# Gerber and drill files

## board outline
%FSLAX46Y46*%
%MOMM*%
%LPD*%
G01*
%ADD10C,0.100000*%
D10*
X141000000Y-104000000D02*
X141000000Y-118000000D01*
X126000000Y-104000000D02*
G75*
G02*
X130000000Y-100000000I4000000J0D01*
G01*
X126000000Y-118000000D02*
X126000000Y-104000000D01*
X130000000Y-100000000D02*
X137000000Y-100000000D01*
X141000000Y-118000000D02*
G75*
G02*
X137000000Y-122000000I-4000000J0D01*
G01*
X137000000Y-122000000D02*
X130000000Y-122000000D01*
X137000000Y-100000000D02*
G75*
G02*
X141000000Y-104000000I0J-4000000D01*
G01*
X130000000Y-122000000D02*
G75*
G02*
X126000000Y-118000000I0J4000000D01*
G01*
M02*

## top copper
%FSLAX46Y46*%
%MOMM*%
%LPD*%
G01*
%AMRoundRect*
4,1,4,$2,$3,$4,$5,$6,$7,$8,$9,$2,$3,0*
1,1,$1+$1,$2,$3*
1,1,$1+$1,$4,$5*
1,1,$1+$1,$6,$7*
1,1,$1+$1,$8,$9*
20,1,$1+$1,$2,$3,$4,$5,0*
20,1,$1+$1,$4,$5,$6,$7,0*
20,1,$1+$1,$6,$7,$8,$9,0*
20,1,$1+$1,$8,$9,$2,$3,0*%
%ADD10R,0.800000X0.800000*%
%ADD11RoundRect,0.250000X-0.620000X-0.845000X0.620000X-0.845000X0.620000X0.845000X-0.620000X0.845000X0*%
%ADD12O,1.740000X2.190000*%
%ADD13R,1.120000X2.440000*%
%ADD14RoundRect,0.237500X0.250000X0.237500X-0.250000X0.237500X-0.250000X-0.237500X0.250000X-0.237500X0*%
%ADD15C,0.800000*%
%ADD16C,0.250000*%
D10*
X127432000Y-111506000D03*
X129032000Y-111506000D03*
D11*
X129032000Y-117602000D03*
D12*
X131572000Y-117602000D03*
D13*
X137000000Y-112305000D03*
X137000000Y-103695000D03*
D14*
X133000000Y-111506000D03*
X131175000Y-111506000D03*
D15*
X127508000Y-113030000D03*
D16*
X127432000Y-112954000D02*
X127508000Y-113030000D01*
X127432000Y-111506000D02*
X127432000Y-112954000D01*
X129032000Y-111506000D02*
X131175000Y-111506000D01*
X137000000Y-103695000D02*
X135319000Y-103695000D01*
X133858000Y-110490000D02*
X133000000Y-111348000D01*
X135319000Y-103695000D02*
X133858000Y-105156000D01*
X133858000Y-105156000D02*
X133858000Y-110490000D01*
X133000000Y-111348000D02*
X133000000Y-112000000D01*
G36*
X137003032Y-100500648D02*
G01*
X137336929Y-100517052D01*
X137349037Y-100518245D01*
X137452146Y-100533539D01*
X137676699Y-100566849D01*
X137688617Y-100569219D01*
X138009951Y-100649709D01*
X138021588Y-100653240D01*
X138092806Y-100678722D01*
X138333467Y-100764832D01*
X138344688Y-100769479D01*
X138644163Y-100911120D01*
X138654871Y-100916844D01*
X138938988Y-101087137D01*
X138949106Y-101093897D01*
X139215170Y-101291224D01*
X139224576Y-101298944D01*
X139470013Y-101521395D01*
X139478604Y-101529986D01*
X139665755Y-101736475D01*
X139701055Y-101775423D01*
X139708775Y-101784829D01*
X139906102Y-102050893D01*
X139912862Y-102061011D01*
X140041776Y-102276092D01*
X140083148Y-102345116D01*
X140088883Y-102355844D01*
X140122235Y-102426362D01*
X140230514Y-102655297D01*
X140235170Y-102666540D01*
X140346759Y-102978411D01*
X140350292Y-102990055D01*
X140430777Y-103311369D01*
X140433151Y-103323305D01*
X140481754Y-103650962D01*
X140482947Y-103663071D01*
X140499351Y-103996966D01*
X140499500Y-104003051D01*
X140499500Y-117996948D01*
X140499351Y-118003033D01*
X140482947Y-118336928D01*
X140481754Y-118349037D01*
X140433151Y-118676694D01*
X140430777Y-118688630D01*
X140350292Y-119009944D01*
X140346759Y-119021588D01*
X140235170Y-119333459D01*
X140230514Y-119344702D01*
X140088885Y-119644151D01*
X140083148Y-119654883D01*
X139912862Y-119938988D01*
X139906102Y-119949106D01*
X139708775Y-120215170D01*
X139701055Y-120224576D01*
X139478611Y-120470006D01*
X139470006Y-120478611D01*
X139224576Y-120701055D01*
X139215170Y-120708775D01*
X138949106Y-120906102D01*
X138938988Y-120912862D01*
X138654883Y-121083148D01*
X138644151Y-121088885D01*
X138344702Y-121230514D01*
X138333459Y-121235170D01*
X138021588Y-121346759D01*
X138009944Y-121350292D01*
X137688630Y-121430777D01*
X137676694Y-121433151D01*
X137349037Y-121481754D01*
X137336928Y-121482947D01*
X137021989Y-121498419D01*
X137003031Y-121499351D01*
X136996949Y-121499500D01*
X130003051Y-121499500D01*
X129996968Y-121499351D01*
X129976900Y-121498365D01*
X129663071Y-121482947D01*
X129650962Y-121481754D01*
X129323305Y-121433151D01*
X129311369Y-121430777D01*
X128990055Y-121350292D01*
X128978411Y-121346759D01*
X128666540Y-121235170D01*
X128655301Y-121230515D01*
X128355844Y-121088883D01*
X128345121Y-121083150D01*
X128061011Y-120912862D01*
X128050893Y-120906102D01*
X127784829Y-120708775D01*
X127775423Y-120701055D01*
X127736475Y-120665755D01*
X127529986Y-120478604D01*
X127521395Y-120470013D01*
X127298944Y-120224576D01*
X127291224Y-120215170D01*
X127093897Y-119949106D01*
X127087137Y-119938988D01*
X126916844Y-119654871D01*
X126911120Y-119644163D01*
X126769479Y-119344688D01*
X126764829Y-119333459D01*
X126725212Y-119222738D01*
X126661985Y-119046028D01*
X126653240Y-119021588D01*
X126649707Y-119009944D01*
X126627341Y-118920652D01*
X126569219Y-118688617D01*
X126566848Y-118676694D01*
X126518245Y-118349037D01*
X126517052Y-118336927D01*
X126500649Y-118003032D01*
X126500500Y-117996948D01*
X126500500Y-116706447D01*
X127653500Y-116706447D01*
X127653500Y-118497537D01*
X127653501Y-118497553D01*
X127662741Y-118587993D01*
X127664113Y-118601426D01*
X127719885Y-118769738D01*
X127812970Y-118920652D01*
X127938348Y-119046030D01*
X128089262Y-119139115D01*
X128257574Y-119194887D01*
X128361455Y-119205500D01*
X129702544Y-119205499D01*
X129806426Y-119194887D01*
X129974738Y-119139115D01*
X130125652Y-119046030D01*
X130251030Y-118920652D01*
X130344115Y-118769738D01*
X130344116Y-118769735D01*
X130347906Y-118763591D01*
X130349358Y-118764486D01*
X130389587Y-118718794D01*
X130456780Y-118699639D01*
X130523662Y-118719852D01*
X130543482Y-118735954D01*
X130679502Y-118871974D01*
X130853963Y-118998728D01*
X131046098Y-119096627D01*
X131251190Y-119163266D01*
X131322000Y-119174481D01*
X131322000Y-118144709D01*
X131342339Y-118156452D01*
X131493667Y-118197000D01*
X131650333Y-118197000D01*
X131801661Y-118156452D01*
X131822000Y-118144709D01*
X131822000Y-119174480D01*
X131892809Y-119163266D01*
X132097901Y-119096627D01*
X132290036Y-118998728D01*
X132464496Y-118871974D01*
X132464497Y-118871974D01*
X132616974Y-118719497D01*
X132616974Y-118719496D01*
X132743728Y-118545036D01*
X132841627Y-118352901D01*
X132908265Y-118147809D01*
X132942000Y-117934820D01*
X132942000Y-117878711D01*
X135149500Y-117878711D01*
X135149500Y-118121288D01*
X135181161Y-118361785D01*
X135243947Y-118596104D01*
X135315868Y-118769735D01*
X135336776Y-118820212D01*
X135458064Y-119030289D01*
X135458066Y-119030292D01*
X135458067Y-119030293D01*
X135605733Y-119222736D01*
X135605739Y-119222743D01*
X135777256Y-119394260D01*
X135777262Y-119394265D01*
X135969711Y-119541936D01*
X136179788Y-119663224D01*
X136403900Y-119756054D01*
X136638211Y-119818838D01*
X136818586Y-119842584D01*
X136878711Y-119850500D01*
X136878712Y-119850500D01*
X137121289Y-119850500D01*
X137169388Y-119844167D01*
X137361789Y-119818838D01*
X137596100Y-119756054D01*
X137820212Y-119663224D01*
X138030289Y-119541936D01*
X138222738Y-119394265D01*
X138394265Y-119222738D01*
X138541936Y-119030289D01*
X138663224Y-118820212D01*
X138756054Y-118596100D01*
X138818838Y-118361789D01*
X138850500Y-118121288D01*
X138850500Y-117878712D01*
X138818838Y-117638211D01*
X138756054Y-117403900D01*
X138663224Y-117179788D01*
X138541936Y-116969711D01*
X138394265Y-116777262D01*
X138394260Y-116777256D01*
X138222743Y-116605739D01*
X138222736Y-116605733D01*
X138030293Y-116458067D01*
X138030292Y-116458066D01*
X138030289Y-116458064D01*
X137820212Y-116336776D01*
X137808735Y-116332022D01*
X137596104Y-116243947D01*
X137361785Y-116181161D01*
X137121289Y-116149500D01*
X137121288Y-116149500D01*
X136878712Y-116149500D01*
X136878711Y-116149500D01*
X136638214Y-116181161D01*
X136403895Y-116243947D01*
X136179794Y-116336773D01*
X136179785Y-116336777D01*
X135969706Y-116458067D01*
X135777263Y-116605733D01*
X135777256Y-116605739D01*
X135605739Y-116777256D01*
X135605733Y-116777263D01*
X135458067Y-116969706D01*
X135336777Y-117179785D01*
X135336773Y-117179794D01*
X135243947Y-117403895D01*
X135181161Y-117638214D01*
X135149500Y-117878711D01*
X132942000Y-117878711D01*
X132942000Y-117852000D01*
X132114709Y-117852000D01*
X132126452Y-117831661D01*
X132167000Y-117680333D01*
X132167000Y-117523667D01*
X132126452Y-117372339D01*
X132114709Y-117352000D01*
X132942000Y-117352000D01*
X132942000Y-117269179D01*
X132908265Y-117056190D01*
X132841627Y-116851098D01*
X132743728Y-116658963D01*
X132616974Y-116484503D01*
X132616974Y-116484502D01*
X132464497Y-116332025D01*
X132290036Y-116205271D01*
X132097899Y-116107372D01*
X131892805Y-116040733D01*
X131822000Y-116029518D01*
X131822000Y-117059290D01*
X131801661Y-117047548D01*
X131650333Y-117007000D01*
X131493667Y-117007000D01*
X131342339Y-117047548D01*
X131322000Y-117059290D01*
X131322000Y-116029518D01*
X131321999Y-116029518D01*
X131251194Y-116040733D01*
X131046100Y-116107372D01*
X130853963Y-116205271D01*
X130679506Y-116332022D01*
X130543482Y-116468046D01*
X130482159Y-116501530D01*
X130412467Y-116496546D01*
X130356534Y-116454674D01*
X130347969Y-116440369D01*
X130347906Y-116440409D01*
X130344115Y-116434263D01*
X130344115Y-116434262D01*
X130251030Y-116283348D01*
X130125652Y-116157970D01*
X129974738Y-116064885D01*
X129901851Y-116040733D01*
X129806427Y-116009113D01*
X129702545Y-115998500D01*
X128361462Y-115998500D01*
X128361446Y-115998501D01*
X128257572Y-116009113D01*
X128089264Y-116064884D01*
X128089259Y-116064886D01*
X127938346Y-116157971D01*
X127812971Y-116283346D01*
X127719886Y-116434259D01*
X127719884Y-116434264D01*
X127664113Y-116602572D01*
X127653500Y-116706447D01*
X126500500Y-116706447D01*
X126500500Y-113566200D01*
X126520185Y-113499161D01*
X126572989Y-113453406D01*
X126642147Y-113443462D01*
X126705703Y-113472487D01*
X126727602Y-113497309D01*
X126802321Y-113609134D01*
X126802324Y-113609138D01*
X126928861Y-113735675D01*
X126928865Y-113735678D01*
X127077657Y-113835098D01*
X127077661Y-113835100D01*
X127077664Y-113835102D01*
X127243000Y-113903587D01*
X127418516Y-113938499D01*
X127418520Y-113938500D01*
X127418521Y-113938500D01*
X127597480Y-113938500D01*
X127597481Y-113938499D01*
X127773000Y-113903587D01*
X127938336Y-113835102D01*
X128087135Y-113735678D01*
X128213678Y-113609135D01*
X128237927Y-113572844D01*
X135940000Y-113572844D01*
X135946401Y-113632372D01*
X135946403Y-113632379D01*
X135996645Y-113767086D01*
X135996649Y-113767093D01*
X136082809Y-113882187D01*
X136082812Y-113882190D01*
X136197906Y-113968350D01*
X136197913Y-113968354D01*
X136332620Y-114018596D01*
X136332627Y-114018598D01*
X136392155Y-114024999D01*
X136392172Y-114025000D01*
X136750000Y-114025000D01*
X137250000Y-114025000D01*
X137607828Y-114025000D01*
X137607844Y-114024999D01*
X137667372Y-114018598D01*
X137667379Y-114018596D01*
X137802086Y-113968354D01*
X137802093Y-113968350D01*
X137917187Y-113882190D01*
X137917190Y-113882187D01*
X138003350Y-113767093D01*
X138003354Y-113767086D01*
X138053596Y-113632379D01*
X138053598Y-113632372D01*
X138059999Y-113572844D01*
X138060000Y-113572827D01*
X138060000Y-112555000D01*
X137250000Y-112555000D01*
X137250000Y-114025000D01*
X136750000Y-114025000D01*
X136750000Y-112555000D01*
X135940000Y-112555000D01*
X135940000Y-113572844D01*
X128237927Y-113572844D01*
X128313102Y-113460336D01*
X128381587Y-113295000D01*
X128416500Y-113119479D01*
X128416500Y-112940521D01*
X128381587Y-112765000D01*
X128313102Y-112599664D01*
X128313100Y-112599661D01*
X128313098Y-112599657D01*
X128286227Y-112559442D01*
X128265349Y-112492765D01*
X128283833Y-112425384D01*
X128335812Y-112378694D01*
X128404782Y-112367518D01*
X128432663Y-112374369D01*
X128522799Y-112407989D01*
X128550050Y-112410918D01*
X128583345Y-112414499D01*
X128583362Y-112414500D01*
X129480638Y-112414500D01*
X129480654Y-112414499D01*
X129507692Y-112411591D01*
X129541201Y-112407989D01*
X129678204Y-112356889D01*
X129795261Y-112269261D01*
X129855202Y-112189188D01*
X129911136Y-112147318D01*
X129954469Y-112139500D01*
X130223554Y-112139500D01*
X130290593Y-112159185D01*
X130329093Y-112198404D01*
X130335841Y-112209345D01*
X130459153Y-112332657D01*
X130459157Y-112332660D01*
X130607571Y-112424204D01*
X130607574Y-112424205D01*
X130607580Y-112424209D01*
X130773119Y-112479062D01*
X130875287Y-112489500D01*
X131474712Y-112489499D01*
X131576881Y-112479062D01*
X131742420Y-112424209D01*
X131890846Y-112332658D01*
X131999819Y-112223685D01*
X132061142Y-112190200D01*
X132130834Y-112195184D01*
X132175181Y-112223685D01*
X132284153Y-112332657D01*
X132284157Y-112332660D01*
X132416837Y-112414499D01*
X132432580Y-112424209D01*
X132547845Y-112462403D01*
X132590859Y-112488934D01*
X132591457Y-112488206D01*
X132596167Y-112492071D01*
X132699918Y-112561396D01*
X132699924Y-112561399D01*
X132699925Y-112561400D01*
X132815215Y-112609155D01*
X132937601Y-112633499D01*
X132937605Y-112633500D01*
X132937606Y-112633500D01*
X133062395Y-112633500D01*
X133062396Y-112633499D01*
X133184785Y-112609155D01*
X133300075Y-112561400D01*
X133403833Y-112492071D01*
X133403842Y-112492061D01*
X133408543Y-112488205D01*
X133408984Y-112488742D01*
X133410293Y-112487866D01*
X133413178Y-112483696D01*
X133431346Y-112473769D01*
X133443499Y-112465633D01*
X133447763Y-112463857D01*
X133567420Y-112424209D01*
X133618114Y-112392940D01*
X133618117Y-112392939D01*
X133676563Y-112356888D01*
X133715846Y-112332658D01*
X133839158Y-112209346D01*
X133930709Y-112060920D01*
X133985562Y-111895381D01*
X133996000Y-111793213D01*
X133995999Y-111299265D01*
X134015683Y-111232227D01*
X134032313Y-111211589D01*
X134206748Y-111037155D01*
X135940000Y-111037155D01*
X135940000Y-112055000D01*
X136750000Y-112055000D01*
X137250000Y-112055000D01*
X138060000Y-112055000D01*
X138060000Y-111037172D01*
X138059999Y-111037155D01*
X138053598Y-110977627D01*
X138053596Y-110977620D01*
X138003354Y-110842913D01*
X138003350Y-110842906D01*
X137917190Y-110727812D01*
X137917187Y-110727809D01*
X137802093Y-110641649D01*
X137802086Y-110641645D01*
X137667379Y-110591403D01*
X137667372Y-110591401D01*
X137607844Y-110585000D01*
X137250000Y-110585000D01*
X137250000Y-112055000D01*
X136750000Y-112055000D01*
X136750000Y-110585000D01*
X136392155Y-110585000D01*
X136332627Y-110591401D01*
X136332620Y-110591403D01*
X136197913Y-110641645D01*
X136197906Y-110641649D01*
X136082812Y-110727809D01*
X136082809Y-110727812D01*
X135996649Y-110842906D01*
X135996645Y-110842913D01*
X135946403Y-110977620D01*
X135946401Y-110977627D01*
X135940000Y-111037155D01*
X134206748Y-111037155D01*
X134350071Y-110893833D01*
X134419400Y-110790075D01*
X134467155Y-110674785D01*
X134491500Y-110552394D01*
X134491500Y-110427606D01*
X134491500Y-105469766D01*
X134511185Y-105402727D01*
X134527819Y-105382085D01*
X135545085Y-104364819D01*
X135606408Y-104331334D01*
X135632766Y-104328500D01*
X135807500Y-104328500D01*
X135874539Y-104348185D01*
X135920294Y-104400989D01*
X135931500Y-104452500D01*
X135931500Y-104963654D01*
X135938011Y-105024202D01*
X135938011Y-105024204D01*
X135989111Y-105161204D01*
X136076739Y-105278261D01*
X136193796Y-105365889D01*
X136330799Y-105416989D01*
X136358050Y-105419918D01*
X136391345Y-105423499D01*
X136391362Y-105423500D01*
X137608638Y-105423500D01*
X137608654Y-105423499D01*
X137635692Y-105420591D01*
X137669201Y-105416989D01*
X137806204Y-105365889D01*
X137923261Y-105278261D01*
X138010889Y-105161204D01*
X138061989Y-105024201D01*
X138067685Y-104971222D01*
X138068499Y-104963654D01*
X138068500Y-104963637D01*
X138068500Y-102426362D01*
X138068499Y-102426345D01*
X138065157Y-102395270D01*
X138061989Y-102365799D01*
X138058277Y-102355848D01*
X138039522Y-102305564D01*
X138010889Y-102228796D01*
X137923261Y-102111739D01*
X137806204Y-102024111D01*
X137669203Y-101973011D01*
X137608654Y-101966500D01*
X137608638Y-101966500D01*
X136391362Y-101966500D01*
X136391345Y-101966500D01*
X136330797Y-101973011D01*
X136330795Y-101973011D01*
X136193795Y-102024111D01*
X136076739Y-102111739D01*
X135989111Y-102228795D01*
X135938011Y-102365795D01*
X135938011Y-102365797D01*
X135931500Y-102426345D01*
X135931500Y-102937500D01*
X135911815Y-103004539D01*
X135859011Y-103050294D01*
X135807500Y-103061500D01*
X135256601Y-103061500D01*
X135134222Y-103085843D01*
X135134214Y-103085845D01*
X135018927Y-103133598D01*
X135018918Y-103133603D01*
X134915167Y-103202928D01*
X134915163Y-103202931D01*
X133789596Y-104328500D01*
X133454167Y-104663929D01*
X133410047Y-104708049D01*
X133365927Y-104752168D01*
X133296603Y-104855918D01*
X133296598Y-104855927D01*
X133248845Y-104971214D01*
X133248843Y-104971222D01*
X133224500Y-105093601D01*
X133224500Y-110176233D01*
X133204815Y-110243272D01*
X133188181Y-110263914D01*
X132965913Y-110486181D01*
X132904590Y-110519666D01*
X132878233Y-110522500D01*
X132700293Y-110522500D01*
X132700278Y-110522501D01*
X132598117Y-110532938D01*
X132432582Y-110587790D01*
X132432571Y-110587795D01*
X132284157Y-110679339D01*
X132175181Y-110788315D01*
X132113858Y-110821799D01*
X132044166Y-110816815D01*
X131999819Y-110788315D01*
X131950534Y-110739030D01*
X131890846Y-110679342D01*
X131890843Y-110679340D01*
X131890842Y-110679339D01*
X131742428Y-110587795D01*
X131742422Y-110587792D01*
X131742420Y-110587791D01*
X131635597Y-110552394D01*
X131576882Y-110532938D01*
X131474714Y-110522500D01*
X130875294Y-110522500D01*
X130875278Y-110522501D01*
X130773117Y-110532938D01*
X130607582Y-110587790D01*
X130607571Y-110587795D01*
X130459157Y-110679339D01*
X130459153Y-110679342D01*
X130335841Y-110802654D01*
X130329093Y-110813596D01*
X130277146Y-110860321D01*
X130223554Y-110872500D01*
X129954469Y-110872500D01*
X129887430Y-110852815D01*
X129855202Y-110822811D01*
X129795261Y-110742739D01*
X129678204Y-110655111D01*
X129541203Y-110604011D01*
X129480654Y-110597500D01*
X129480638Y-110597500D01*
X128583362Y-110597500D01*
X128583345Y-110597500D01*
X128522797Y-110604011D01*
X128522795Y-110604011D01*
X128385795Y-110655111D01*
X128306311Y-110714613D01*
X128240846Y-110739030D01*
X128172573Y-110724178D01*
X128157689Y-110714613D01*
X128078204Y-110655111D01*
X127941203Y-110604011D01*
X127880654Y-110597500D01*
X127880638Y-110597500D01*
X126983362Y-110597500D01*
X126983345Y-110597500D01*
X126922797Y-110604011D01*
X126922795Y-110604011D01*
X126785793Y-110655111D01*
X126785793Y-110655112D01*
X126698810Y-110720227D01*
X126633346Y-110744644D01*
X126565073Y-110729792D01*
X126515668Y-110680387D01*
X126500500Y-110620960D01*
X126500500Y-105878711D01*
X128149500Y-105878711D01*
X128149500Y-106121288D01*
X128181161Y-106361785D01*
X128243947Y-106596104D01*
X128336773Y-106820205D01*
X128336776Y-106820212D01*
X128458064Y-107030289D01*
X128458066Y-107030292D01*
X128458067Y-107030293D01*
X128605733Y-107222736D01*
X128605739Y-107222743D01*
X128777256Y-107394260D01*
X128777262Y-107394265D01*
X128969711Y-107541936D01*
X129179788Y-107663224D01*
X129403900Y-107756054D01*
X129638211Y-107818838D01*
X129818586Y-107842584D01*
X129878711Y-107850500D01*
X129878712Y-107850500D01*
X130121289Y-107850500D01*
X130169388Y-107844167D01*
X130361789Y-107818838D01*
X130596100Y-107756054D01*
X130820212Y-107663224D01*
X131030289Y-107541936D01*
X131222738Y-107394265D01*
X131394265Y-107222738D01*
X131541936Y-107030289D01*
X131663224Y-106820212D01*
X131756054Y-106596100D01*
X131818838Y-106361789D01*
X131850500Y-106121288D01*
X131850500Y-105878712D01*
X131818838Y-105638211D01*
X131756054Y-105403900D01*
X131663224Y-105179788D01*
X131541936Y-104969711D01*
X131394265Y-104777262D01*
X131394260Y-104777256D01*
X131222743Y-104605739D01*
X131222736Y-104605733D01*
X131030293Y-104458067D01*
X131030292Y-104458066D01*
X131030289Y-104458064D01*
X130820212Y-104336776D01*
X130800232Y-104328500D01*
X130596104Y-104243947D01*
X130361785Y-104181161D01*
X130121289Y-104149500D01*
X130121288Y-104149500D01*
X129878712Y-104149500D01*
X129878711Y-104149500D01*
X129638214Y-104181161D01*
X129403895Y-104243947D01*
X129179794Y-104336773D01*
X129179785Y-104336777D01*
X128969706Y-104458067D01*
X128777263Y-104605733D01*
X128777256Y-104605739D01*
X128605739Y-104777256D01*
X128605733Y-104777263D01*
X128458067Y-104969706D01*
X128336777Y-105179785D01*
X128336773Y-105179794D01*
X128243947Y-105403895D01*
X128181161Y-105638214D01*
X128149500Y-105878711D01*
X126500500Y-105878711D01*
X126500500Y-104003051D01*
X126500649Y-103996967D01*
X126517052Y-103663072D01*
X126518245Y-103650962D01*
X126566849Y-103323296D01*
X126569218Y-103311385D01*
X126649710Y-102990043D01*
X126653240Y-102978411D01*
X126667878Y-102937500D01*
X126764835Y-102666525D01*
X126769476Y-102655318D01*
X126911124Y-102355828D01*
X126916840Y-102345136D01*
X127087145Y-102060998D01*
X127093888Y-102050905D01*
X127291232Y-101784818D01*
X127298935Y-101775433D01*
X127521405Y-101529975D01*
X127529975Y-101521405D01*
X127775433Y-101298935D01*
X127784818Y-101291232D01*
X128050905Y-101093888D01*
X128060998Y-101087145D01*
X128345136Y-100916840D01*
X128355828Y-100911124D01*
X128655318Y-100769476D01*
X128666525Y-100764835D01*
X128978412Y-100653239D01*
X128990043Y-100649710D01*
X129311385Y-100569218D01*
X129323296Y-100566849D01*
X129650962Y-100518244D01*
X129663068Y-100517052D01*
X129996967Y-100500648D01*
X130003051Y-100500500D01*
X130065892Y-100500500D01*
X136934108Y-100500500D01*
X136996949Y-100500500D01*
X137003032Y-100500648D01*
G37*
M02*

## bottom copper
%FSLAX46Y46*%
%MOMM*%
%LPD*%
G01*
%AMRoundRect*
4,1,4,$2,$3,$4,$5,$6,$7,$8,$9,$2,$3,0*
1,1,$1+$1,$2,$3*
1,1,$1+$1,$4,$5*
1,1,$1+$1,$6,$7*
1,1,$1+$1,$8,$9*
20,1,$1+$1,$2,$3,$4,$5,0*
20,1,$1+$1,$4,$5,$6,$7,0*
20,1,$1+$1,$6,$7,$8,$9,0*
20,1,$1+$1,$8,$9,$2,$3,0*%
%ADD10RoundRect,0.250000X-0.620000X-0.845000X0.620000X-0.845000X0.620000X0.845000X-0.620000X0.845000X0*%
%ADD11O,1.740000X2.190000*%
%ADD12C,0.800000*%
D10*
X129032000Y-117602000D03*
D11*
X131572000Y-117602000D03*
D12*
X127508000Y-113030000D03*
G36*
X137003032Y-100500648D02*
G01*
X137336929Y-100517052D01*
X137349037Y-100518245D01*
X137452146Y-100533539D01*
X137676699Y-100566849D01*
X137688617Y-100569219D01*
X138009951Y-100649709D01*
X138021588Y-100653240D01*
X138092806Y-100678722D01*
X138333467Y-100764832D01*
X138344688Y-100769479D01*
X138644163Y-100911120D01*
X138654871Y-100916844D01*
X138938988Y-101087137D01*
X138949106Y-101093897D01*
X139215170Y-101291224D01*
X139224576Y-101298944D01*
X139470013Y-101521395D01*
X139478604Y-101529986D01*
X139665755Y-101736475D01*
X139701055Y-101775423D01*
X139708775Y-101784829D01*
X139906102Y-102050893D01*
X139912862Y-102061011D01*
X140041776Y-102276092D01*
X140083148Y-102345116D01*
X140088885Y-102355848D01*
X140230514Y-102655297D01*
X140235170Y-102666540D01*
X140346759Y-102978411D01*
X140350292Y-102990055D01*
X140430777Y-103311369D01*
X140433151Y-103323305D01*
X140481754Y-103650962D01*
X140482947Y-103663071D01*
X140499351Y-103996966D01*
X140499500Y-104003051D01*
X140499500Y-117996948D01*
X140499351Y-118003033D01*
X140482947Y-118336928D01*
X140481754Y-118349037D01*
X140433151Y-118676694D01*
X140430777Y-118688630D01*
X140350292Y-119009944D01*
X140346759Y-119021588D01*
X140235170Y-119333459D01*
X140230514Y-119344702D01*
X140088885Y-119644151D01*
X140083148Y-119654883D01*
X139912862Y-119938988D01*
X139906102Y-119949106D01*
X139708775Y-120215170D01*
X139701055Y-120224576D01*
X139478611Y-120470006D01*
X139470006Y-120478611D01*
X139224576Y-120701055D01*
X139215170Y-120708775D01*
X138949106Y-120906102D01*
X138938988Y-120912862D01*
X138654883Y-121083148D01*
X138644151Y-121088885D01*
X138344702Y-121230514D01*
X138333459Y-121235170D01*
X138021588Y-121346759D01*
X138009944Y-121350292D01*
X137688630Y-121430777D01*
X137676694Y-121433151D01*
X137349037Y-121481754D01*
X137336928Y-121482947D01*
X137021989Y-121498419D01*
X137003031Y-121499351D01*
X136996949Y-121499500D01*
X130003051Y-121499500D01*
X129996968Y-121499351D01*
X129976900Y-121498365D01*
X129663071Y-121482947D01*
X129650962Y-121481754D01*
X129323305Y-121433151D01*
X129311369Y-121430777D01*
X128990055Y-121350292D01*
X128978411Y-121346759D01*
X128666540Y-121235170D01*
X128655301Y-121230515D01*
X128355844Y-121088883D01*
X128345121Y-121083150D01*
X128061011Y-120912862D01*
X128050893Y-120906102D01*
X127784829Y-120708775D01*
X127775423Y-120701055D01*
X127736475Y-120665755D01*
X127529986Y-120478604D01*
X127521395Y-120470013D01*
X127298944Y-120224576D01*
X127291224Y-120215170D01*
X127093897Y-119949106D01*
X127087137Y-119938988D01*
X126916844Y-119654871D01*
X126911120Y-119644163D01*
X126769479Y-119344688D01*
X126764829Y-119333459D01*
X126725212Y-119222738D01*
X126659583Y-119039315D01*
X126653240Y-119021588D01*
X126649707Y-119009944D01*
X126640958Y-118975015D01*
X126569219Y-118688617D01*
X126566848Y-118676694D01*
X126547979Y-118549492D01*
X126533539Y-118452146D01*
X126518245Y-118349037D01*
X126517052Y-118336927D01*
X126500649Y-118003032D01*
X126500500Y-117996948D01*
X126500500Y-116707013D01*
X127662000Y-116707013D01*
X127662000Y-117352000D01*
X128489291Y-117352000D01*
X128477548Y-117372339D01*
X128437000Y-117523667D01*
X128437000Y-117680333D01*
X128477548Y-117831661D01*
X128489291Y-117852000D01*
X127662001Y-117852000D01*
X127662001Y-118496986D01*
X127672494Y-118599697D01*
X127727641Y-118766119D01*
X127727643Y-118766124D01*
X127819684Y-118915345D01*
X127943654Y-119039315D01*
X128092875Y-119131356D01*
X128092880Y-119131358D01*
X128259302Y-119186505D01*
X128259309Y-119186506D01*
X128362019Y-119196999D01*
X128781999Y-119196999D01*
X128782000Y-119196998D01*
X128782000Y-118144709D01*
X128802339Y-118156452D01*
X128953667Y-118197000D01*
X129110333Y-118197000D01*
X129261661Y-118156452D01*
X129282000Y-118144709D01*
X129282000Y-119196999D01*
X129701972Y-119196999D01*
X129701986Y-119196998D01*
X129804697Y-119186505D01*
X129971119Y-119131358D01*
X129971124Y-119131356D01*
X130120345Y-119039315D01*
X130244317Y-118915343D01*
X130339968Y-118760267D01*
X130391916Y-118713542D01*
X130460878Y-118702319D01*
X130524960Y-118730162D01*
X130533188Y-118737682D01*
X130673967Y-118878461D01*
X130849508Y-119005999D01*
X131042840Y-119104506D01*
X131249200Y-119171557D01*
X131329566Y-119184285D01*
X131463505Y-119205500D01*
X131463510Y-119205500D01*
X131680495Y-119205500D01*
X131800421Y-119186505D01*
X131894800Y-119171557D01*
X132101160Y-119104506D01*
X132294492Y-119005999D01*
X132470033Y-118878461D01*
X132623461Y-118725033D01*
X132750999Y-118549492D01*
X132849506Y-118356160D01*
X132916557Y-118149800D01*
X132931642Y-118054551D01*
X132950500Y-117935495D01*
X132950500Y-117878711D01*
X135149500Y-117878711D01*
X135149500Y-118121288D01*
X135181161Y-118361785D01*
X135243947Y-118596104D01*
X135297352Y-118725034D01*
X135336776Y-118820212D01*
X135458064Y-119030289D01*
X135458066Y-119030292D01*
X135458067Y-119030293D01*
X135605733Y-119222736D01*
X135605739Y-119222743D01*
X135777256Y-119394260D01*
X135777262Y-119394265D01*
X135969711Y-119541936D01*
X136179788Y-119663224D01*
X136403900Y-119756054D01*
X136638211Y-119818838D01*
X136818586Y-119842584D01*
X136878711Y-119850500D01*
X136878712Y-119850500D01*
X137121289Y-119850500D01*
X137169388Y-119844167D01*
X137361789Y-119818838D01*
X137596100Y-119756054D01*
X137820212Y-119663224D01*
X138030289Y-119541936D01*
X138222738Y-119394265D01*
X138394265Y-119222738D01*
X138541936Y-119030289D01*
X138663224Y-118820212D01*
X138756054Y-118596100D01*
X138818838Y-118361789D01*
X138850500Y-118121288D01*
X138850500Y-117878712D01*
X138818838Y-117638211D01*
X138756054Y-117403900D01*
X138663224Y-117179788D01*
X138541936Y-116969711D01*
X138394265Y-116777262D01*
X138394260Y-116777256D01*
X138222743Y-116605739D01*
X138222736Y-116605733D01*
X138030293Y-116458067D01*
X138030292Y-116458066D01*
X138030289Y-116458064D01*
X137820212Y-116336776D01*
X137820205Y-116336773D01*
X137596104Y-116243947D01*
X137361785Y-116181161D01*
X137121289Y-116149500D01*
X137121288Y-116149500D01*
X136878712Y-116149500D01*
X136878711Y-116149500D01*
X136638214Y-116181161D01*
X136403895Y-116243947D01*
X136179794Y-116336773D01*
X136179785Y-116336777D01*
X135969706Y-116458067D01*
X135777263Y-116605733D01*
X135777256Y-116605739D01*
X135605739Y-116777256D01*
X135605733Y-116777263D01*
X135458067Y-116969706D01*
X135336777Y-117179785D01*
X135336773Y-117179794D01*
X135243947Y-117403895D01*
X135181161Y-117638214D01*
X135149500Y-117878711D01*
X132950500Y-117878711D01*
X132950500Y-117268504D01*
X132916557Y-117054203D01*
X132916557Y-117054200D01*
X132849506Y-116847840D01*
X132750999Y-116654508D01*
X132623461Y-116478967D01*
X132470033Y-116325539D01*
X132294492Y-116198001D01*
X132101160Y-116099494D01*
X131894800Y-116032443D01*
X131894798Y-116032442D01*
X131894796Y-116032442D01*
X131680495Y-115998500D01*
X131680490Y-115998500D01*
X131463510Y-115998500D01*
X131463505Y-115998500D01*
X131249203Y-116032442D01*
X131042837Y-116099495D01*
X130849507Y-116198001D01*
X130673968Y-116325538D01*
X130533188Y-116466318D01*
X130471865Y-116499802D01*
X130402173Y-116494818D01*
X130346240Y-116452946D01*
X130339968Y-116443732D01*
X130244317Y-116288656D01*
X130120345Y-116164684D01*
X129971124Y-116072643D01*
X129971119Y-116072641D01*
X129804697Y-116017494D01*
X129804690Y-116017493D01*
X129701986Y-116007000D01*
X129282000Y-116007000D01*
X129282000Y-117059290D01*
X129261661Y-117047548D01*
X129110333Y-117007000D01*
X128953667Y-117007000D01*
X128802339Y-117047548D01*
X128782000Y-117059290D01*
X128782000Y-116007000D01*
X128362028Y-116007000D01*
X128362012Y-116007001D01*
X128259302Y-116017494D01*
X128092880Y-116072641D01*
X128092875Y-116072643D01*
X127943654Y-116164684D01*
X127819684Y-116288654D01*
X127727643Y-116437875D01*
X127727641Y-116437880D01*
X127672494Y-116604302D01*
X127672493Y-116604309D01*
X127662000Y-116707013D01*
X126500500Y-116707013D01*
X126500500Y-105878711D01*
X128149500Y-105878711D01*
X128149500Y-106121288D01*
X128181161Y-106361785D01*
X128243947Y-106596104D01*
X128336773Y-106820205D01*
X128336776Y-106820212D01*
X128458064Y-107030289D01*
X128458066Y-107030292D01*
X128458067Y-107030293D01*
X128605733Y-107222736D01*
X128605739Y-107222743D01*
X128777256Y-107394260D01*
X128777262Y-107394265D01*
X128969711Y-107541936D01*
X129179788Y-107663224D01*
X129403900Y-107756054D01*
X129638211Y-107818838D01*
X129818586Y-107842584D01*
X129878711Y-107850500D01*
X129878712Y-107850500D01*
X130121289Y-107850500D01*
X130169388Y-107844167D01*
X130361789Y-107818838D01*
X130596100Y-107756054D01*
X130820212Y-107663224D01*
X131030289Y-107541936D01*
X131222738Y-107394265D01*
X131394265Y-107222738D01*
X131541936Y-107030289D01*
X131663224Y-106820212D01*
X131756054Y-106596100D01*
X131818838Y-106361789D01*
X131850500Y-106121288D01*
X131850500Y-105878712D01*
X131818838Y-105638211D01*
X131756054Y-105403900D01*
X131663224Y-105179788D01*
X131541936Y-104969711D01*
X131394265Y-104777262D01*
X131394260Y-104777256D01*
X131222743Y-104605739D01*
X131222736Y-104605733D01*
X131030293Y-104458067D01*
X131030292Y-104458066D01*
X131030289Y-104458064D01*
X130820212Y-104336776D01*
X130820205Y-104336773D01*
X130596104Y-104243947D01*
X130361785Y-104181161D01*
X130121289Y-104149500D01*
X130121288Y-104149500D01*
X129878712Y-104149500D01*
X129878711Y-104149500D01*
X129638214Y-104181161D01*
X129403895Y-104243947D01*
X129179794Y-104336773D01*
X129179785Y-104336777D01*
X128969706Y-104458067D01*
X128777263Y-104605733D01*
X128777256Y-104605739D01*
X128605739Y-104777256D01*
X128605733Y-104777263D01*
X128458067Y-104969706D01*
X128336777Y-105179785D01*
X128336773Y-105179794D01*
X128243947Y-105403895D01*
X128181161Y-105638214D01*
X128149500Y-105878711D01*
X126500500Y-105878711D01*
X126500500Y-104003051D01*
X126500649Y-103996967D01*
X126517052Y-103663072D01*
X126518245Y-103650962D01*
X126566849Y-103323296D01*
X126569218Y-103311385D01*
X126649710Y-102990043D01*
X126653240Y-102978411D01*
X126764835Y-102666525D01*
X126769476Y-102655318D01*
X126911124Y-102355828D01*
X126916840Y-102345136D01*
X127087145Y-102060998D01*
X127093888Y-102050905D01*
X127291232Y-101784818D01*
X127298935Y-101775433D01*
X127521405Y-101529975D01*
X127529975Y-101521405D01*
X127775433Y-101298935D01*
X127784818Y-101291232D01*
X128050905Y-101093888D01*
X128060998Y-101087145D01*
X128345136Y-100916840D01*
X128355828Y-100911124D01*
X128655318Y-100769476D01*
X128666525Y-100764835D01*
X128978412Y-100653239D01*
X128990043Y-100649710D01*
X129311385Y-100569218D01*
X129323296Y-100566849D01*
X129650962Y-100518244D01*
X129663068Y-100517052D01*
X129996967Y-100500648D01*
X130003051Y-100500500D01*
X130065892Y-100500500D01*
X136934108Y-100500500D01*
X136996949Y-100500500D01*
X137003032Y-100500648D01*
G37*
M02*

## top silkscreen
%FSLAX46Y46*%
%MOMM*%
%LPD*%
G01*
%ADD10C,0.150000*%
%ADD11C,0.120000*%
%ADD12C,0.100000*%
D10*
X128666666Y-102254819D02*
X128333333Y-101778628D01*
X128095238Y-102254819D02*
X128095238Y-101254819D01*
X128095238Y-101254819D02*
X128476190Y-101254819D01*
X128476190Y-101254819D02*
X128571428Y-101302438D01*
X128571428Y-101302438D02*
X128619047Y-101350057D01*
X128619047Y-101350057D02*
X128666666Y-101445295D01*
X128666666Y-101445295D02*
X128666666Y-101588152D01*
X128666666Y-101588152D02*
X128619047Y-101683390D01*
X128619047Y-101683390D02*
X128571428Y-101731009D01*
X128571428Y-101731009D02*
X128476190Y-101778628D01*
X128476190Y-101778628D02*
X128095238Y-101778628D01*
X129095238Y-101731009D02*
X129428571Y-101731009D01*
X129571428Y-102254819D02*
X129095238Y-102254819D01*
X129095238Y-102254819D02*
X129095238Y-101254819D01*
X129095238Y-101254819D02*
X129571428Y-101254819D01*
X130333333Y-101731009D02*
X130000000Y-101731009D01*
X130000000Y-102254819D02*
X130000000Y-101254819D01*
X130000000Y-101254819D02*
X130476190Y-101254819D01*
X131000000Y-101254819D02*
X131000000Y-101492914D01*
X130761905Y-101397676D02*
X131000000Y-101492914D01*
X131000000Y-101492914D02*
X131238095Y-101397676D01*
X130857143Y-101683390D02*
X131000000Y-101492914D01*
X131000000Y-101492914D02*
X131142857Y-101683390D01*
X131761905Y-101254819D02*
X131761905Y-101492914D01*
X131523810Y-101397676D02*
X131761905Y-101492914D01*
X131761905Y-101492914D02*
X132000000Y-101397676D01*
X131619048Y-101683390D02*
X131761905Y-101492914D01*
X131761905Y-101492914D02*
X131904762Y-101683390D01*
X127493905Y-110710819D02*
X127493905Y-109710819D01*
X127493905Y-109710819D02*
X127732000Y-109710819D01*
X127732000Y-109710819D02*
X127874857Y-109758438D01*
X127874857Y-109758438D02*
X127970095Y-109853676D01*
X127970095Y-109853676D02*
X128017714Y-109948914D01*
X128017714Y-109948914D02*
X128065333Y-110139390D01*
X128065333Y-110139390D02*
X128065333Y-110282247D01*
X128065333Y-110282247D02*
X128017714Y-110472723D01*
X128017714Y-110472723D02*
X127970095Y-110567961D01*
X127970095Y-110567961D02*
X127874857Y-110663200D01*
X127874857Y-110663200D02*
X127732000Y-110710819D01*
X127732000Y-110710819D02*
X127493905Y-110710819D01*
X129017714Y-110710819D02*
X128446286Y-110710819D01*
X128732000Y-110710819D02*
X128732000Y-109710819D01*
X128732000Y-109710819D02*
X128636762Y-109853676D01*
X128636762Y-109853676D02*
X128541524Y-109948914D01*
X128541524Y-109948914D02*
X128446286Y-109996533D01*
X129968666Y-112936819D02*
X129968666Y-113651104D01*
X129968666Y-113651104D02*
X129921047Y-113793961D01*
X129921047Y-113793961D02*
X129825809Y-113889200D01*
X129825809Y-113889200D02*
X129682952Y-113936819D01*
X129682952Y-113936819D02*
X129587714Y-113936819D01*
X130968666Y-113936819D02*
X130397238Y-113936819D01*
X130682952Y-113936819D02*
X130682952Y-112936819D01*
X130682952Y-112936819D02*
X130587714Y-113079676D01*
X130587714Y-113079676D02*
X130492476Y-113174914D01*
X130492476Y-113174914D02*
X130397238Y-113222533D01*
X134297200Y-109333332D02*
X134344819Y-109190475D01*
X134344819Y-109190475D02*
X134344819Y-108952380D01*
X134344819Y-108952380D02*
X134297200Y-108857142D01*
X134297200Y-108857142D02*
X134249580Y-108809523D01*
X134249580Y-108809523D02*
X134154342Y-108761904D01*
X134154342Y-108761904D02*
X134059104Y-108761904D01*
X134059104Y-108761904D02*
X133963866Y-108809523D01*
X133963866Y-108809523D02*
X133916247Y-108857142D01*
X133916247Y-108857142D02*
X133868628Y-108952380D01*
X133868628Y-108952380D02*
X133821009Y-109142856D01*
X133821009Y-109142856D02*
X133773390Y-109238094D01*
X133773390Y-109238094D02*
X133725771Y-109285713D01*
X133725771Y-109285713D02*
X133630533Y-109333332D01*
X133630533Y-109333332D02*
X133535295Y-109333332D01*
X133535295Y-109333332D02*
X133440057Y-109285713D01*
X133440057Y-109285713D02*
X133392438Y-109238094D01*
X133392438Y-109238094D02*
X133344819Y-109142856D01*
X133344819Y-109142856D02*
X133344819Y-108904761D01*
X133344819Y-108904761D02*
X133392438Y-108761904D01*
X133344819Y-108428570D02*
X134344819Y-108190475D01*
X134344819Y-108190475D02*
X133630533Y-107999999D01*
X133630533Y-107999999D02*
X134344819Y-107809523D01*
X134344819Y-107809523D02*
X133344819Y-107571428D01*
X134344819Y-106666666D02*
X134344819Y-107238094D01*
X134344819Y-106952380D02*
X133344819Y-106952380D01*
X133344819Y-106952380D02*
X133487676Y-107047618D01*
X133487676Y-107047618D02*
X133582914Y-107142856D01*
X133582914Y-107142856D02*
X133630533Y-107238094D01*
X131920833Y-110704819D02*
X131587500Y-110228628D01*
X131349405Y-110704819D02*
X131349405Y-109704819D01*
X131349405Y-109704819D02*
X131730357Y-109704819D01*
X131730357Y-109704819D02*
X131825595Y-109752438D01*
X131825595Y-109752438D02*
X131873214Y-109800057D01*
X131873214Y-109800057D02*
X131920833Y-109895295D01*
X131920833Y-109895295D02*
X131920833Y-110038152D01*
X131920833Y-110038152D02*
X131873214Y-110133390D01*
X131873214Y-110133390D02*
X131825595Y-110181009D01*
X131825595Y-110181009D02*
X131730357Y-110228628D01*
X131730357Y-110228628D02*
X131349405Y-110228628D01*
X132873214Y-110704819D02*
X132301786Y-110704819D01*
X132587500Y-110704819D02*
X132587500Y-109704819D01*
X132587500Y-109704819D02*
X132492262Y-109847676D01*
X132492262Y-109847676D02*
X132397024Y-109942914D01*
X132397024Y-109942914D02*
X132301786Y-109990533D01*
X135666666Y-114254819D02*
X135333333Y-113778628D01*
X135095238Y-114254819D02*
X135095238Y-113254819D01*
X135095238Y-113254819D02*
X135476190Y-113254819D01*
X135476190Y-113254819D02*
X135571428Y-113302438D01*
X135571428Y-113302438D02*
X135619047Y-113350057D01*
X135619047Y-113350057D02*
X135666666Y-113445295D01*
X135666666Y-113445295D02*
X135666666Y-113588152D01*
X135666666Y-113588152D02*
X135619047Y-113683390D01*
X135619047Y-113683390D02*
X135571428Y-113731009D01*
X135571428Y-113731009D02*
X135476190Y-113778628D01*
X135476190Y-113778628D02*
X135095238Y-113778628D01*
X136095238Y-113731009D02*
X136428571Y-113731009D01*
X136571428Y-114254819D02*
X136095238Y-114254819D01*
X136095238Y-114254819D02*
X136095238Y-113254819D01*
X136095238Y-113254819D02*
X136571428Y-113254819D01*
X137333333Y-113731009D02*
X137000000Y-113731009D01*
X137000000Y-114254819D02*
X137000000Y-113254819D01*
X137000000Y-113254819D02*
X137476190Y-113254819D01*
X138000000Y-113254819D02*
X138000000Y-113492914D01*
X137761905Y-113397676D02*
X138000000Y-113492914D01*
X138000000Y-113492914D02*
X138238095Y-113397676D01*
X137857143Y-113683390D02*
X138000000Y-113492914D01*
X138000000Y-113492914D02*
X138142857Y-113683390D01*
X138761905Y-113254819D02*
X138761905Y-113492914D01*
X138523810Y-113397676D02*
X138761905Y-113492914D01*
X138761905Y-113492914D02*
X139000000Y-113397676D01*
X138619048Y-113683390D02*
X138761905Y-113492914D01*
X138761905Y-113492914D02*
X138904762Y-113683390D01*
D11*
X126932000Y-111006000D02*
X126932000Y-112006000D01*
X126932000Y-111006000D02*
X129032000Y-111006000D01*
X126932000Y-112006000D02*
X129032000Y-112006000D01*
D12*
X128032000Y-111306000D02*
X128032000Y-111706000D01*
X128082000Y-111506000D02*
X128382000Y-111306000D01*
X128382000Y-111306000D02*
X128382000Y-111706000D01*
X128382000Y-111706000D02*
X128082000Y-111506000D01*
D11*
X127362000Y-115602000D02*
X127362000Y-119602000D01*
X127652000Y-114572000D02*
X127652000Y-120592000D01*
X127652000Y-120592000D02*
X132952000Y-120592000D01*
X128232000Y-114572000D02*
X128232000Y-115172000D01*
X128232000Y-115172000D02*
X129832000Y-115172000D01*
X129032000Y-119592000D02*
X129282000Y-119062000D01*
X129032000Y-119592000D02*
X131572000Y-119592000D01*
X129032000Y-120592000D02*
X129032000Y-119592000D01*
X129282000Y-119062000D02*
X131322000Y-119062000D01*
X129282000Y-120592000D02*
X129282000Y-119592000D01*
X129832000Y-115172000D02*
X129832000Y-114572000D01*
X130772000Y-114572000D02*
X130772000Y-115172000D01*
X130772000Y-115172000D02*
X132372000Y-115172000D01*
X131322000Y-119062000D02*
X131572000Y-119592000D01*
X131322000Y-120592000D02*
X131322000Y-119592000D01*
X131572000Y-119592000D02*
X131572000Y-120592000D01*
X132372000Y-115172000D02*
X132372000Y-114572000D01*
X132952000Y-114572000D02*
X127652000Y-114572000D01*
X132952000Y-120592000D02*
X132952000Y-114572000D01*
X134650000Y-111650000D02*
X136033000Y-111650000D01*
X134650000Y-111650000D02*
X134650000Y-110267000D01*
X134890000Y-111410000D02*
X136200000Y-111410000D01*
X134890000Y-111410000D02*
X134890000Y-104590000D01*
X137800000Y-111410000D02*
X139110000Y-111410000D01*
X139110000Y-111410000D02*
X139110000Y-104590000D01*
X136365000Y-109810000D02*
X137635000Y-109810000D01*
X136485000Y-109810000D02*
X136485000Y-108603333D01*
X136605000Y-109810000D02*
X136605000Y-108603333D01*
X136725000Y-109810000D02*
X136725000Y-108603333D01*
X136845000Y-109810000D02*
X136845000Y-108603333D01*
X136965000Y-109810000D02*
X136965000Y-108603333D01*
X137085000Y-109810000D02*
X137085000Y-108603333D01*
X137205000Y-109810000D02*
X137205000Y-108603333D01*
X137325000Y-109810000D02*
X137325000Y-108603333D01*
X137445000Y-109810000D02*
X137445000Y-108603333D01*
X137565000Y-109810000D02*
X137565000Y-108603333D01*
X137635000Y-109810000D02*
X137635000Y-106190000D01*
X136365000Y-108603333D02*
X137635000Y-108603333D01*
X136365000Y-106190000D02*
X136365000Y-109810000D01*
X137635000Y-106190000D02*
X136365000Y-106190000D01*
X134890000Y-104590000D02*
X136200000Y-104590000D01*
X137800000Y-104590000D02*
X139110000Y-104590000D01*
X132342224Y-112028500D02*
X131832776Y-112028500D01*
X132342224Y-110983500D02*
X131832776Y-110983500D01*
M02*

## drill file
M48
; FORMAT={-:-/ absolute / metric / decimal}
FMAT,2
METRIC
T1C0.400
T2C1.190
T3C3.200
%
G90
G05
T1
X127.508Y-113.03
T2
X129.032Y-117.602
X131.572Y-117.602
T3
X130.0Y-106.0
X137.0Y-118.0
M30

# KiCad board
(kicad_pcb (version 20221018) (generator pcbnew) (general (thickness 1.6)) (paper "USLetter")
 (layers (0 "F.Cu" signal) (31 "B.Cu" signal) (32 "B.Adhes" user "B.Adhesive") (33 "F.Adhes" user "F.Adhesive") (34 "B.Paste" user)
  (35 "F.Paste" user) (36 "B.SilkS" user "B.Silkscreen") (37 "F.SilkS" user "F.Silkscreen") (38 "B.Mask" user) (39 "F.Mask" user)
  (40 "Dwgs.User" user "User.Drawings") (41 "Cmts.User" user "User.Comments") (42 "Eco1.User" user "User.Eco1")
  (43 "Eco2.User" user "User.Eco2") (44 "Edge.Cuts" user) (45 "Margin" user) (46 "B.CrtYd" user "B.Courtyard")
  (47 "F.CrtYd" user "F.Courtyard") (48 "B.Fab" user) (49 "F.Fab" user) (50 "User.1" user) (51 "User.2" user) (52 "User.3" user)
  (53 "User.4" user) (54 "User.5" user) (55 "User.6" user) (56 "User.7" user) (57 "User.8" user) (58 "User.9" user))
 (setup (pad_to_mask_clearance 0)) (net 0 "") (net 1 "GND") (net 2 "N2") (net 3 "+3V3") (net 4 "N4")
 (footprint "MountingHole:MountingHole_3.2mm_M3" (layer "F.Cu") (at 130 106)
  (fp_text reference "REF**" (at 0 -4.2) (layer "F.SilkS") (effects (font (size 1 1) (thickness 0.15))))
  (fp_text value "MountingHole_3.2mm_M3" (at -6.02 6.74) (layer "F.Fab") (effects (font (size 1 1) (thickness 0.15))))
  (pad "" np_thru_hole circle (at 0 0) (size 3.2 3.2) (drill 3.2) (layers "*.Cu" "*.Mask")))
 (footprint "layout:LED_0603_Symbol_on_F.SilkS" (layer "F.Cu") (at 128.232 111.506)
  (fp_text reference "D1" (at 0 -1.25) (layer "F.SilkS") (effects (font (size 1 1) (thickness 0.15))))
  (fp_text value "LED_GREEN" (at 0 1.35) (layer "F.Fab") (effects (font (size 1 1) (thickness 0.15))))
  (fp_line (start -1.3 -0.5) (end -1.3 0.5) (stroke (width 0.12) (type solid)) (layer "F.SilkS"))
  (fp_line (start -1.3 -0.5) (end 0.8 -0.5) (stroke (width 0.12) (type solid)) (layer "F.SilkS"))
  (fp_line (start -1.3 0.5) (end 0.8 0.5) (stroke (width 0.12) (type solid)) (layer "F.SilkS"))
  (fp_line (start -0.2 -0.2) (end -0.2 0.2) (stroke (width 0.1) (type solid)) (layer "F.SilkS"))
  (fp_line (start -0.15 0) (end 0.15 -0.2) (stroke (width 0.1) (type solid)) (layer "F.SilkS"))
  (fp_line (start 0.15 -0.2) (end 0.15 0.2) (stroke (width 0.1) (type solid)) (layer "F.SilkS"))
  (fp_line (start 0.15 0.2) (end -0.15 0) (stroke (width 0.1) (type solid)) (layer "F.SilkS"))
  (pad "1" smd rect (at -0.8 0 180) (size 0.8 0.8) (layers "F.Cu" "F.Paste" "F.Mask") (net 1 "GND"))
  (pad "2" smd rect (at 0.8 0 180) (size 0.8 0.8) (layers "F.Cu" "F.Paste" "F.Mask") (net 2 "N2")))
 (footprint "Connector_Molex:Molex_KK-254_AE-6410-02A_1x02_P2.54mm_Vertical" (layer "F.Cu") (at 129.032 117.602)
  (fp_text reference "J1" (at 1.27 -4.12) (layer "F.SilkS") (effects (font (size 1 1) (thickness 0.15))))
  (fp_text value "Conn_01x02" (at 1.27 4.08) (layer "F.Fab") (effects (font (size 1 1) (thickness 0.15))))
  (fp_line (start -1.67 -2) (end -1.67 2) (stroke (width 0.12) (type solid)) (layer "F.SilkS"))
  (fp_line (start -1.38 -3.03) (end -1.38 2.99) (stroke (width 0.12) (type solid)) (layer "F.SilkS"))
  (fp_line (start -1.38 2.99) (end 3.92 2.99) (stroke (width 0.12) (type solid)) (layer "F.SilkS"))
  (fp_line (start -0.8 -3.03) (end -0.8 -2.43) (stroke (width 0.12) (type solid)) (layer "F.SilkS"))
  (fp_line (start -0.8 -2.43) (end 0.8 -2.43) (stroke (width 0.12) (type solid)) (layer "F.SilkS"))
  (fp_line (start 0 1.99) (end 0.25 1.46) (stroke (width 0.12) (type solid)) (layer "F.SilkS"))
  (fp_line (start 0 1.99) (end 2.54 1.99) (stroke (width 0.12) (type solid)) (layer "F.SilkS"))
  (fp_line (start 0 2.99) (end 0 1.99) (stroke (width 0.12) (type solid)) (layer "F.SilkS"))
  (fp_line (start 0.25 1.46) (end 2.29 1.46) (stroke (width 0.12) (type solid)) (layer "F.SilkS"))
  (fp_line (start 0.25 2.99) (end 0.25 1.99) (stroke (width 0.12) (type solid)) (layer "F.SilkS"))
  (fp_line (start 0.8 -2.43) (end 0.8 -3.03) (stroke (width 0.12) (type solid)) (layer "F.SilkS"))
  (fp_line (start 1.74 -3.03) (end 1.74 -2.43) (stroke (width 0.12) (type solid)) (layer "F.SilkS"))
  (fp_line (start 1.74 -2.43) (end 3.34 -2.43) (stroke (width 0.12) (type solid)) (layer "F.SilkS"))
  (fp_line (start 2.29 1.46) (end 2.54 1.99) (stroke (width 0.12) (type solid)) (layer "F.SilkS"))
  (fp_line (start 2.29 2.99) (end 2.29 1.99) (stroke (width 0.12) (type solid)) (layer "F.SilkS"))
  (fp_line (start 2.54 1.99) (end 2.54 2.99) (stroke (width 0.12) (type solid)) (layer "F.SilkS"))
  (fp_line (start 3.34 -2.43) (end 3.34 -3.03) (stroke (width 0.12) (type solid)) (layer "F.SilkS"))
  (fp_line (start 3.92 -3.03) (end -1.38 -3.03) (stroke (width 0.12) (type solid)) (layer "F.SilkS"))
  (fp_line (start 3.92 2.99) (end 3.92 -3.03) (stroke (width 0.12) (type solid)) (layer "F.SilkS"))
  (pad "1" thru_hole roundrect (at 0 0) (size 1.74 2.19) (drill 1.19) (layers "*.Cu" "*.Mask") (roundrect_rratio 0.143678) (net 1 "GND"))
  (pad "2" thru_hole oval (at 2.54 0) (size 1.74 2.19) (drill 1.19) (layers "*.Cu" "*.Mask") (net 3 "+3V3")))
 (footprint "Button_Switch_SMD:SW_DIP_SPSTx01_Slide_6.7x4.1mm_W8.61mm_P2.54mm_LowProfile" (layer "F.Cu") (at 137 108 90)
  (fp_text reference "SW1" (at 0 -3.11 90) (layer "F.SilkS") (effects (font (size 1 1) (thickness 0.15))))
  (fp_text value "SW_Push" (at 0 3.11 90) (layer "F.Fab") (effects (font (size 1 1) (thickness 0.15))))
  (fp_line (start -3.65 -2.35) (end -3.65 -0.967) (stroke (width 0.12) (type solid)) (layer "F.SilkS"))
  (fp_line (start -3.65 -2.35) (end -2.267 -2.35) (stroke (width 0.12) (type solid)) (layer "F.SilkS"))
  (fp_line (start -3.41 -2.11) (end -3.41 -0.8) (stroke (width 0.12) (type solid)) (layer "F.SilkS"))
  (fp_line (start -3.41 -2.11) (end 3.41 -2.11) (stroke (width 0.12) (type solid)) (layer "F.SilkS"))
  (fp_line (start -3.41 0.8) (end -3.41 2.11) (stroke (width 0.12) (type solid)) (layer "F.SilkS"))
  (fp_line (start -3.41 2.11) (end 3.41 2.11) (stroke (width 0.12) (type solid)) (layer "F.SilkS"))
  (fp_line (start -1.81 -0.635) (end -1.81 0.635) (stroke (width 0.12) (type solid)) (layer "F.SilkS"))
  (fp_line (start -1.81 -0.515) (end -0.603333 -0.515) (stroke (width 0.12) (type solid)) (layer "F.SilkS"))
  (fp_line (start -1.81 -0.395) (end -0.603333 -0.395) (stroke (width 0.12) (type solid)) (layer "F.SilkS"))
  (fp_line (start -1.81 -0.275) (end -0.603333 -0.275) (stroke (width 0.12) (type solid)) (layer "F.SilkS"))
  (fp_line (start -1.81 -0.155) (end -0.603333 -0.155) (stroke (width 0.12) (type solid)) (layer "F.SilkS"))
  (fp_line (start -1.81 -0.035) (end -0.603333 -0.035) (stroke (width 0.12) (type solid)) (layer "F.SilkS"))
  (fp_line (start -1.81 0.085) (end -0.603333 0.085) (stroke (width 0.12) (type solid)) (layer "F.SilkS"))
  (fp_line (start -1.81 0.205) (end -0.603333 0.205) (stroke (width 0.12) (type solid)) (layer "F.SilkS"))
  (fp_line (start -1.81 0.325) (end -0.603333 0.325) (stroke (width 0.12) (type solid)) (layer "F.SilkS"))
  (fp_line (start -1.81 0.445) (end -0.603333 0.445) (stroke (width 0.12) (type solid)) (layer "F.SilkS"))
  (fp_line (start -1.81 0.565) (end -0.603333 0.565) (stroke (width 0.12) (type solid)) (layer "F.SilkS"))
  (fp_line (start -1.81 0.635) (end 1.81 0.635) (stroke (width 0.12) (type solid)) (layer "F.SilkS"))
  (fp_line (start -0.603333 -0.635) (end -0.603333 0.635) (stroke (width 0.12) (type solid)) (layer "F.SilkS"))
  (fp_line (start 1.81 -0.635) (end -1.81 -0.635) (stroke (width 0.12) (type solid)) (layer "F.SilkS"))
  (fp_line (start 1.81 0.635) (end 1.81 -0.635) (stroke (width 0.12) (type solid)) (layer "F.SilkS"))
  (fp_line (start 3.41 -2.11) (end 3.41 -0.8) (stroke (width 0.12) (type solid)) (layer "F.SilkS"))
  (fp_line (start 3.41 0.8) (end 3.41 2.11) (stroke (width 0.12) (type solid)) (layer "F.SilkS"))
  (pad "1" smd rect (at -4.305 0 90) (size 2.44 1.12) (layers "F.Cu" "F.Paste" "F.Mask") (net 3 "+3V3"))
  (pad "2" smd rect (at 4.305 0 90) (size 2.44 1.12) (layers "F.Cu" "F.Paste" "F.Mask") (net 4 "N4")))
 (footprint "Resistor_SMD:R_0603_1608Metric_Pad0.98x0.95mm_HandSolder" (layer "F.Cu") (at 132.0875 111.506 180)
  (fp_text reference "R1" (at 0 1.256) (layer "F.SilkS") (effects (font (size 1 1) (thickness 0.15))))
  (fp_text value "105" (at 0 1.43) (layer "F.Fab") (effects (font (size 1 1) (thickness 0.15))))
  (fp_line (start -0.254724 -0.5225) (end 0.254724 -0.5225) (stroke (width 0.12) (type solid)) (layer "F.SilkS"))
  (fp_line (start -0.254724 0.5225) (end 0.254724 0.5225) (stroke (width 0.12) (type solid)) (layer "F.SilkS"))
  (pad "1" smd roundrect (at -0.9125 0 180) (size 0.975 0.95) (layers "F.Cu" "F.Paste" "F.Mask") (roundrect_rratio 0.25) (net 4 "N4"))
  (pad "2" smd roundrect (at 0.9125 0 180) (size 0.975 0.95) (layers "F.Cu" "F.Paste" "F.Mask") (roundrect_rratio 0.25) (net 2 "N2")))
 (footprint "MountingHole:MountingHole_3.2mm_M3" (layer "F.Cu") (at 137 118)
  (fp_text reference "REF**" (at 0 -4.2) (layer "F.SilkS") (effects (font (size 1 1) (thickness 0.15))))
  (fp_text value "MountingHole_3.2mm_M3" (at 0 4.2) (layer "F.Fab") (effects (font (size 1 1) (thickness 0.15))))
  (pad "" np_thru_hole circle (at 0 0) (size 3.2 3.2) (drill 3.2) (layers "F&B.Cu" "*.Mask")))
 (gr_line (start 141 104) (end 141 118) (stroke (width 0.1) (type default)) (layer "Edge.Cuts"))
 (gr_arc (start 126 104) (mid 127.171573 101.171573) (end 130 100) (stroke (width 0.1) (type default)) (layer "Edge.Cuts"))
 (gr_line (start 126 118) (end 126 104) (stroke (width 0.1) (type default)) (layer "Edge.Cuts"))
 (gr_line (start 130 100) (end 137 100) (stroke (width 0.1) (type default)) (layer "Edge.Cuts"))
 (gr_arc (start 141 118) (mid 139.828427 120.828427) (end 137 122) (stroke (width 0.1) (type default)) (layer "Edge.Cuts"))
 (gr_line (start 137 122) (end 130 122) (stroke (width 0.1) (type default)) (layer "Edge.Cuts"))
 (gr_arc (start 137 100) (mid 139.828427 101.171573) (end 141 104) (stroke (width 0.1) (type default)) (layer "Edge.Cuts"))
 (gr_arc (start 130 122) (mid 127.171573 120.828427) (end 126 118) (stroke (width 0.1) (type default)) (layer "Edge.Cuts"))
 (segment (start 127.432 112.954) (end 127.508 113.03) (width 0.25) (layer "F.Cu") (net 1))
 (segment (start 127.432 111.506) (end 127.432 112.954) (width 0.25) (layer "F.Cu") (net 1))
 (via (at 127.508 113.03) (size 0.8) (drill 0.4) (layers "F.Cu" "B.Cu") (free) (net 1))
 (segment (start 129.032 111.506) (end 131.175 111.506) (width 0.25) (layer "F.Cu") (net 2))
 (segment (start 137 103.695) (end 135.319 103.695) (width 0.25) (layer "F.Cu") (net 4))
 (segment (start 133.858 110.49) (end 133 111.348) (width 0.25) (layer "F.Cu") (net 4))
 (segment (start 135.319 103.695) (end 133.858 105.156) (width 0.25) (layer "F.Cu") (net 4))
 (segment (start 133.858 105.156) (end 133.858 110.49) (width 0.25) (layer "F.Cu") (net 4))
 (segment (start 133 111.348) (end 133 112) (width 0.25) (layer "F.Cu") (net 4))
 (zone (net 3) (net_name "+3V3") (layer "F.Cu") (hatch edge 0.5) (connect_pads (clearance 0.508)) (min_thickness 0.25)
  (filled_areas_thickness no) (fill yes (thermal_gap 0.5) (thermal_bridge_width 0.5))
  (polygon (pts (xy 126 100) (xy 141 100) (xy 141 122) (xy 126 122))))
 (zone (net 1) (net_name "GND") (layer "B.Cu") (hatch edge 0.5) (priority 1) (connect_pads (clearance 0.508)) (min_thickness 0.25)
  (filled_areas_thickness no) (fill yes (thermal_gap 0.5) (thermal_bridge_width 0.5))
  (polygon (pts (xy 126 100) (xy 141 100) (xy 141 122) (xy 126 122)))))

